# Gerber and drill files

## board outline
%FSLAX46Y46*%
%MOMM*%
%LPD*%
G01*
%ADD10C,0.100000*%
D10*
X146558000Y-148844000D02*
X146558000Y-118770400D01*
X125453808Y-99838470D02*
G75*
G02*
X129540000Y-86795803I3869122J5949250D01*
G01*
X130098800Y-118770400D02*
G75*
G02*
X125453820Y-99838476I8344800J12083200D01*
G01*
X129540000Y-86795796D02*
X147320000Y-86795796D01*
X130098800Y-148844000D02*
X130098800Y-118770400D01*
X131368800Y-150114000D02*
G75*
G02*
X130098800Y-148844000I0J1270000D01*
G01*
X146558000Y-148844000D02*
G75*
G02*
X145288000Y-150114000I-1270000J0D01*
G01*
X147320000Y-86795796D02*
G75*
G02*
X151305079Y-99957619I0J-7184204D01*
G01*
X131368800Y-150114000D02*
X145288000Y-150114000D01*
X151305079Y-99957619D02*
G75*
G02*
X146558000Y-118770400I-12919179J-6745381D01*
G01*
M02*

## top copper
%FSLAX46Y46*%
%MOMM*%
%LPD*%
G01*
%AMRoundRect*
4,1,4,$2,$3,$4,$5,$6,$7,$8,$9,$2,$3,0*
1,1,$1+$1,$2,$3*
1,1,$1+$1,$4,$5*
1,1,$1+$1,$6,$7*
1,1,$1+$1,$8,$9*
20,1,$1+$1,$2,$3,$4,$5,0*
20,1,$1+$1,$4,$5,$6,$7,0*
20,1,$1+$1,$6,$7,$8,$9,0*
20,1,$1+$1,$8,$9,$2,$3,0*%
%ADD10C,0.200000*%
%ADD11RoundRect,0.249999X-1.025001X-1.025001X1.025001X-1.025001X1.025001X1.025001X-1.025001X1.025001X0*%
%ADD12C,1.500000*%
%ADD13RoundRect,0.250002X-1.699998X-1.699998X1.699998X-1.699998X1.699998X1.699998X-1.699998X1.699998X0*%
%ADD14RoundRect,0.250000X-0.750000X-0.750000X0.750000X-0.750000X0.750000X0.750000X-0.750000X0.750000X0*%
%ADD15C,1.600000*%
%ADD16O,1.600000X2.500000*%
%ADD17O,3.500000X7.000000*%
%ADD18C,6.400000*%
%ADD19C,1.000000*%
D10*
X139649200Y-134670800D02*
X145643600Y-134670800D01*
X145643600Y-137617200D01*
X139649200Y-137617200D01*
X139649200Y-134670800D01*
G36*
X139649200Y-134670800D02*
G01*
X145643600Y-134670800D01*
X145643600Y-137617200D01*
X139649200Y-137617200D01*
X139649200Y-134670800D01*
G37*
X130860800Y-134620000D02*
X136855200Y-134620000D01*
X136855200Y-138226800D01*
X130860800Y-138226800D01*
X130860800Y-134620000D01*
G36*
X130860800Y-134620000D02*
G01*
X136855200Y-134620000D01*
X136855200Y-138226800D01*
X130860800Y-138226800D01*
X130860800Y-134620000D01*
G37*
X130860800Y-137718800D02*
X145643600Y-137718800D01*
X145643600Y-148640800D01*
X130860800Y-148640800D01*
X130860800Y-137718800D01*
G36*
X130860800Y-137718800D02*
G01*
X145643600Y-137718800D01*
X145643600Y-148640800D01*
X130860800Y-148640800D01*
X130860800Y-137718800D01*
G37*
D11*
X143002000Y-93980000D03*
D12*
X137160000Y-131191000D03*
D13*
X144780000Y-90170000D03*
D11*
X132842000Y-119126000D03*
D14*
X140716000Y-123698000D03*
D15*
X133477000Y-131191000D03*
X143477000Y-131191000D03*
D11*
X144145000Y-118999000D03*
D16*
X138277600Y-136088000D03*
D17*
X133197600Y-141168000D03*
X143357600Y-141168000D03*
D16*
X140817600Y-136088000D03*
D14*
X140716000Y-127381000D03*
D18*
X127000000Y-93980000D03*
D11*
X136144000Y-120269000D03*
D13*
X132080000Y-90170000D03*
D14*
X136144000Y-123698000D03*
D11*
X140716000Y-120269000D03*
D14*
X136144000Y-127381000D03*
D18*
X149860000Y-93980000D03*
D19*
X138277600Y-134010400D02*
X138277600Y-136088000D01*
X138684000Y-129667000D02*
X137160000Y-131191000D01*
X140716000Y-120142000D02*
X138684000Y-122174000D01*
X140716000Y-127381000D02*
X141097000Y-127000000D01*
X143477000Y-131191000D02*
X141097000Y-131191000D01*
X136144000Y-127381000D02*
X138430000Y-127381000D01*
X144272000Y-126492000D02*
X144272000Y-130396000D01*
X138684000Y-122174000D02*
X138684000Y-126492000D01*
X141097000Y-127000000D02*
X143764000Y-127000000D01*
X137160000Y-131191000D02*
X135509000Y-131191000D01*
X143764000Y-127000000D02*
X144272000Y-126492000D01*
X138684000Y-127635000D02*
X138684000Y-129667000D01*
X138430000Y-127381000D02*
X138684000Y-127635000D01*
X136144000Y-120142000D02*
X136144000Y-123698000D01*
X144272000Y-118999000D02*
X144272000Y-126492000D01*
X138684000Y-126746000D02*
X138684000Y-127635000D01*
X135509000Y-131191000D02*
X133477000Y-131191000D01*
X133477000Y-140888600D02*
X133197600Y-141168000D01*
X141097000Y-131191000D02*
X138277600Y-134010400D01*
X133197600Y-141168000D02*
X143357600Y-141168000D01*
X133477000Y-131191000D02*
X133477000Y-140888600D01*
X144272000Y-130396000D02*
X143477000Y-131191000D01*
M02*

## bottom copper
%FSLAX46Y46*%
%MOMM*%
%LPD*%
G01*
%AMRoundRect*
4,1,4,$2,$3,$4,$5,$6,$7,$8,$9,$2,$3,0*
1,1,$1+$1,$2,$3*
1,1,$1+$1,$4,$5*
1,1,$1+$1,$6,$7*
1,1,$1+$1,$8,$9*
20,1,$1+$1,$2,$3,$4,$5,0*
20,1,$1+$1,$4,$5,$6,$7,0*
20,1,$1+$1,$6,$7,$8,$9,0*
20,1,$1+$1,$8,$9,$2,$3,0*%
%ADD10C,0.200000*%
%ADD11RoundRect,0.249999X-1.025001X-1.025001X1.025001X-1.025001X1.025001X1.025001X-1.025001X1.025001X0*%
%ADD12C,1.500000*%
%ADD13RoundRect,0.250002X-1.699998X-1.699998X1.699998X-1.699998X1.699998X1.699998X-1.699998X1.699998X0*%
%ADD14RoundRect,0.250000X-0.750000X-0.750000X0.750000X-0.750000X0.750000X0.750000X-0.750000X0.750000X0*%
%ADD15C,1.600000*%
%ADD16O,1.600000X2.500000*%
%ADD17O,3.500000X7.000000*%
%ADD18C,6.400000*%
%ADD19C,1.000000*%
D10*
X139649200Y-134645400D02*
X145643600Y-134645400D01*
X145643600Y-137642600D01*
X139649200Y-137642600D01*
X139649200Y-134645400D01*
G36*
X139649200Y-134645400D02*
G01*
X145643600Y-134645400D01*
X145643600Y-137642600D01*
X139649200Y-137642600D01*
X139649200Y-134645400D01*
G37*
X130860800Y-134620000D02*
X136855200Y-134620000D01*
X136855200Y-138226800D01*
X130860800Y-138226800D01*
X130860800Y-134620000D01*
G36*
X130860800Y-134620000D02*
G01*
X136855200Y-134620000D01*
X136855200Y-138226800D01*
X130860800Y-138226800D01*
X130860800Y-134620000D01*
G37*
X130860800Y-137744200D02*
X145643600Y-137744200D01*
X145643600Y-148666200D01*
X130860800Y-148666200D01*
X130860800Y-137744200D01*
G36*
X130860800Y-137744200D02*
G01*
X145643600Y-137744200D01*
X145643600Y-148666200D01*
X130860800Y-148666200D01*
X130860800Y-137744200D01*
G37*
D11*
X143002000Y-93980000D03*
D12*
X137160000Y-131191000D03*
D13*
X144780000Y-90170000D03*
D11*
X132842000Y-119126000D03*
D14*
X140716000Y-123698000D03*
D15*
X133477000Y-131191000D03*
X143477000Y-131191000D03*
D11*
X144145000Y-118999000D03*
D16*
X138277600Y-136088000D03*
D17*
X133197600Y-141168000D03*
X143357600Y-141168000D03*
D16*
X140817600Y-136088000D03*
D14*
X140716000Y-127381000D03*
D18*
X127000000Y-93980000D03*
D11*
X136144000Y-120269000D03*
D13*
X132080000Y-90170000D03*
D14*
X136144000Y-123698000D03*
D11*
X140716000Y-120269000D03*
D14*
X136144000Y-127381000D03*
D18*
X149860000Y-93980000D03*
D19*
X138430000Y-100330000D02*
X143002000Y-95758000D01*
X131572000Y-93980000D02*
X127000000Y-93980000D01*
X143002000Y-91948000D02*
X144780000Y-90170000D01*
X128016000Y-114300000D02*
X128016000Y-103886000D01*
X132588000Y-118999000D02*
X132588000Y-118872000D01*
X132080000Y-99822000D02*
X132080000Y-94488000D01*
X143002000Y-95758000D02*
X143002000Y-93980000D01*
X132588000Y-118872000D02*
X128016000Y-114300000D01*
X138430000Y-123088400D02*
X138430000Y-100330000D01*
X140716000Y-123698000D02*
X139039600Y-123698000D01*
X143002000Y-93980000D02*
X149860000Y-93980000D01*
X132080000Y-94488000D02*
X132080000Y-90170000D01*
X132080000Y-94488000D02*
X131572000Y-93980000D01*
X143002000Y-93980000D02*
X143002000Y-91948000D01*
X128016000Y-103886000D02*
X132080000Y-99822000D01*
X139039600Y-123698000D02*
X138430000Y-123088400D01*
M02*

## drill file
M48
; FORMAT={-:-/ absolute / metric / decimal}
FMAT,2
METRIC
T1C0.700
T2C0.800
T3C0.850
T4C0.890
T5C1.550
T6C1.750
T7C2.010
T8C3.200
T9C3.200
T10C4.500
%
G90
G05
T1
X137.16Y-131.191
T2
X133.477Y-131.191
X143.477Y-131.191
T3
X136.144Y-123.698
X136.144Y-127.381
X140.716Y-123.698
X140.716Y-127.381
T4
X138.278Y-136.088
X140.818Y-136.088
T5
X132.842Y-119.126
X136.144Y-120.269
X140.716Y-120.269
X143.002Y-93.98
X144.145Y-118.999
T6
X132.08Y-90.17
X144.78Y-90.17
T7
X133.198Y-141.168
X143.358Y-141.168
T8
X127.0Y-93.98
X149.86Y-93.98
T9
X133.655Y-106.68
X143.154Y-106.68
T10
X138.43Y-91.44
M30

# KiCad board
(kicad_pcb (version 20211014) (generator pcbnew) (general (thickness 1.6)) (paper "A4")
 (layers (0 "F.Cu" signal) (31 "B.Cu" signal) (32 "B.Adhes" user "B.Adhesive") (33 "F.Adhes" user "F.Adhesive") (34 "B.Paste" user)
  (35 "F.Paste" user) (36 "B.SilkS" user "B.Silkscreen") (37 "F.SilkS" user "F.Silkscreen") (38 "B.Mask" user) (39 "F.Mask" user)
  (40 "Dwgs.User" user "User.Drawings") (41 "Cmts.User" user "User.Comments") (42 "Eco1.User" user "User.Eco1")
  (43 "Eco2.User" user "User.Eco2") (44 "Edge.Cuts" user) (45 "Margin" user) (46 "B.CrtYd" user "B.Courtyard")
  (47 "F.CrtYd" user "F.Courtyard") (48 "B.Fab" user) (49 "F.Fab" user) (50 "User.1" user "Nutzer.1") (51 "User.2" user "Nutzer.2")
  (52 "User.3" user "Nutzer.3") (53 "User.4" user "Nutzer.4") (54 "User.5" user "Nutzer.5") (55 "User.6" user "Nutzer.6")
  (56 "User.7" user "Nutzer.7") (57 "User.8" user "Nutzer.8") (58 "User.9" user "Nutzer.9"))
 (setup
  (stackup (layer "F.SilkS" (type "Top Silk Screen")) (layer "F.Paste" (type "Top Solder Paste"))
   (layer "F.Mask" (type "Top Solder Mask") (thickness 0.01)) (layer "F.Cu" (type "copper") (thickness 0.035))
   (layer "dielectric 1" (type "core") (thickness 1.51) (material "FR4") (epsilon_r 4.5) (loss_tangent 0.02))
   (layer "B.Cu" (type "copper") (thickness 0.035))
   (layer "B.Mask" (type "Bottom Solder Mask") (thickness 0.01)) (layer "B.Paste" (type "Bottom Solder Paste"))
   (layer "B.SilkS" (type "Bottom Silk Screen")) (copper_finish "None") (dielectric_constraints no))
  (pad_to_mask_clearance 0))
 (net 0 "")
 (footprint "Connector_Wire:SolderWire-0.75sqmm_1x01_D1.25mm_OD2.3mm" (layer "F.Cu") (at 143.002 93.98)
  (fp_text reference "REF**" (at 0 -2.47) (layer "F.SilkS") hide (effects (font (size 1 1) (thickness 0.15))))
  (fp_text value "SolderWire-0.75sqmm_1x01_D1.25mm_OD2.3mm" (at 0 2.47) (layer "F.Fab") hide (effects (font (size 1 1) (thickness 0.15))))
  (pad "1" thru_hole roundrect (at 0 0) (size 2.55 2.55) (drill 1.55) (layers *.Cu *.Mask) (roundrect_rratio 0.098039)))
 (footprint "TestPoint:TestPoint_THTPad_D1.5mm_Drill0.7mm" (layer "F.Cu") (at 137.16 131.191)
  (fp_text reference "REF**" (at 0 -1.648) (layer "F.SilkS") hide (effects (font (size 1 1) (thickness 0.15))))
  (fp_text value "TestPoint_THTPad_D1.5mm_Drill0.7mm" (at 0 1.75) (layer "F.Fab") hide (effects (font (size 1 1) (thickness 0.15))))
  (pad "1" thru_hole circle (at 0 0) (size 1.5 1.5) (drill 0.7) (layers *.Cu *.Mask)))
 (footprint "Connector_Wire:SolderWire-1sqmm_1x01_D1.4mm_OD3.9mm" (layer "F.Cu") (at 144.78 90.17)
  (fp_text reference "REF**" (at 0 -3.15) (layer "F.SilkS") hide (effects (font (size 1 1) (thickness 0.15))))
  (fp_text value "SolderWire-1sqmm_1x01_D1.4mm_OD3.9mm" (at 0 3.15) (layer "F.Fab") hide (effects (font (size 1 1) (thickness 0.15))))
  (pad "1" thru_hole roundrect (at 0 0) (size 3.9 3.9) (drill 1.75) (layers *.Cu *.Mask) (roundrect_rratio 0.064103)))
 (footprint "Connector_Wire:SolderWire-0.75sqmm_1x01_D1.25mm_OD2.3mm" (layer "F.Cu") (at 132.842 119.126)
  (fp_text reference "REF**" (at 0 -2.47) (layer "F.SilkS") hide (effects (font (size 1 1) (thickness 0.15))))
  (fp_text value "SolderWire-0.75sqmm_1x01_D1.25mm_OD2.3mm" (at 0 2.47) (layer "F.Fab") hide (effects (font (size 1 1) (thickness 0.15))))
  (pad "1" thru_hole roundrect (at 0 0) (size 2.55 2.55) (drill 1.55) (layers *.Cu *.Mask) (roundrect_rratio 0.098039)))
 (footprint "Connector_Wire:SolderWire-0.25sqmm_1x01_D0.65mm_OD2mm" (layer "F.Cu") (at 140.716 123.698)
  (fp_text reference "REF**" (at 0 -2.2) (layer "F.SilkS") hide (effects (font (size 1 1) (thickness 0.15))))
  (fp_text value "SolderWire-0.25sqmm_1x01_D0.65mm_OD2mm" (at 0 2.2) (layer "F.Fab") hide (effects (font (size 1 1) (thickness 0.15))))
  (pad "1" thru_hole roundrect (at 0 0) (size 2 2) (drill 0.85) (layers *.Cu *.Mask) (roundrect_rratio 0.125)))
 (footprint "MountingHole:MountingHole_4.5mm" (layer "F.Cu") (at 138.43 91.44)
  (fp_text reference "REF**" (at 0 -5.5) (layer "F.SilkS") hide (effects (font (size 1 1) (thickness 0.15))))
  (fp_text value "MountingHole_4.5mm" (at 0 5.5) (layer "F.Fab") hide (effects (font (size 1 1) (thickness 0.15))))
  (pad "" np_thru_hole circle (at 0 0) (size 4.5 4.5) (drill 4.5) (layers *.Cu *.Mask)))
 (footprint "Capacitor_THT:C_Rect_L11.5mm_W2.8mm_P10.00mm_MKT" (layer "F.Cu") (at 133.477 131.191)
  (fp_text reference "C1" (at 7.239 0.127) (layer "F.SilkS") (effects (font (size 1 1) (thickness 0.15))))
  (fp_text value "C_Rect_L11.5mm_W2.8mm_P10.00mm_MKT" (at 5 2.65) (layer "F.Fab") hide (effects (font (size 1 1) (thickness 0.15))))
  (pad "1" thru_hole circle (at 0 0) (size 1.6 1.6) (drill 0.8) (layers *.Cu *.Mask))
  (pad "2" thru_hole circle (at 10 0) (size 1.6 1.6) (drill 0.8) (layers *.Cu *.Mask)))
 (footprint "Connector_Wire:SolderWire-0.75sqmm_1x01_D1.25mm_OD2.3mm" (layer "F.Cu") (at 144.145 118.999)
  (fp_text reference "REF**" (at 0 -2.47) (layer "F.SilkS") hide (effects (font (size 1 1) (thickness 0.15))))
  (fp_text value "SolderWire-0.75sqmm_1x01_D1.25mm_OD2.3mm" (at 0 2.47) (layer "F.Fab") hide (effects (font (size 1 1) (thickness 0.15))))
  (pad "1" thru_hole roundrect (at 0 0) (size 2.55 2.55) (drill 1.55) (layers *.Cu *.Mask) (roundrect_rratio 0.098039)))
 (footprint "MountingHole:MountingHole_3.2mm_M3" (layer "F.Cu") (at 143.1544 106.68)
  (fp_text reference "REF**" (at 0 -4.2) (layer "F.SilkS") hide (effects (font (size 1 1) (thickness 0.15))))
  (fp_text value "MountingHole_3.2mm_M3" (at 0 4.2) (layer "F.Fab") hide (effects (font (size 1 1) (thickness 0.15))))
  (pad "" np_thru_hole circle (at 0 0) (size 3.2 3.2) (drill 3.2) (layers *.Cu *.Mask)))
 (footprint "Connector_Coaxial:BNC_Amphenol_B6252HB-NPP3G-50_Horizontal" (layer "F.Cu") (at 138.2776 136.088 180)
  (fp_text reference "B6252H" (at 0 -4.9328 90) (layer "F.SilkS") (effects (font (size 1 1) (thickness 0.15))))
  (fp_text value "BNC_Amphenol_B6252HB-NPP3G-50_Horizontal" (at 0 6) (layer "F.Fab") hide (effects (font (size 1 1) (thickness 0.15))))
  (pad "1" thru_hole oval (at 0 0 180) (size 1.6 2.5) (drill 0.89) (layers *.Cu *.Mask))
  (pad "2" thru_hole oval (at 5.08 -5.08 180) (size 3.5 7) (drill 2.01) (layers *.Cu *.Mask))
  (pad "2" thru_hole oval (at -5.08 -5.08 180) (size 3.5 7) (drill 2.01) (layers *.Cu *.Mask))
  (pad "2" thru_hole oval (at -2.54 0 180) (size 1.6 2.5) (drill 0.89) (layers *.Cu *.Mask)))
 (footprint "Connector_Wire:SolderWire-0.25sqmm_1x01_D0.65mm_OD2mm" (layer "F.Cu") (at 140.716 127.381)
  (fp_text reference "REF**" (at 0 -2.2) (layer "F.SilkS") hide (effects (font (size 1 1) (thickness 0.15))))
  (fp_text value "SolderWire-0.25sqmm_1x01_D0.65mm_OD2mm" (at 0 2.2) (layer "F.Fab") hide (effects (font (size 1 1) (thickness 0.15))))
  (pad "1" thru_hole roundrect (at 0 0) (size 2 2) (drill 0.85) (layers *.Cu *.Mask) (roundrect_rratio 0.125)))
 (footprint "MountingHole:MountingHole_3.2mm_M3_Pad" (layer "F.Cu") (at 127 93.98)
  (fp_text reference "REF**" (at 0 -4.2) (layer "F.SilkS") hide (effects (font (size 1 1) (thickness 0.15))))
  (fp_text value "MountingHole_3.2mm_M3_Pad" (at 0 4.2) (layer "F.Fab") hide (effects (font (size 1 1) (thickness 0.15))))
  (pad "1" thru_hole circle (at 0 0) (size 6.4 6.4) (drill 3.2) (layers *.Cu *.Mask)))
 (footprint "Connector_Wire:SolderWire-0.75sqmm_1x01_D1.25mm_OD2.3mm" (layer "F.Cu") (at 136.144 120.269)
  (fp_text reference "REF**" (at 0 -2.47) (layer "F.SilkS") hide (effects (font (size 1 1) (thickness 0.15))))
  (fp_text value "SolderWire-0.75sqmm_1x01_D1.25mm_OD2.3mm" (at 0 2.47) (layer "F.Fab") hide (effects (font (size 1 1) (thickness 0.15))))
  (pad "1" thru_hole roundrect (at 0 0) (size 2.55 2.55) (drill 1.55) (layers *.Cu *.Mask) (roundrect_rratio 0.098039)))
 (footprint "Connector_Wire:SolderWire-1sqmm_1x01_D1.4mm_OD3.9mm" (layer "F.Cu") (at 132.08 90.17)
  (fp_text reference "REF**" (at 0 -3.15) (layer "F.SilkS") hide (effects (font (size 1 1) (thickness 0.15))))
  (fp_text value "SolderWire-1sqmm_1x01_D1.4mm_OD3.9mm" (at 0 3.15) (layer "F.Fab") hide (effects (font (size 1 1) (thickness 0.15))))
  (pad "1" thru_hole roundrect (at 0 0) (size 3.9 3.9) (drill 1.75) (layers *.Cu *.Mask) (roundrect_rratio 0.064103)))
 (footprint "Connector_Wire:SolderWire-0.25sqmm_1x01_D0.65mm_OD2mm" (layer "F.Cu") (at 136.144 123.698)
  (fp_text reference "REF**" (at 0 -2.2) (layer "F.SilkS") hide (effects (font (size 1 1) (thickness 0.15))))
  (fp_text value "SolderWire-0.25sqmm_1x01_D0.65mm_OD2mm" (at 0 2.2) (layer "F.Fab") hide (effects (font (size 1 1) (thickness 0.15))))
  (pad "1" thru_hole roundrect (at 0 0) (size 2 2) (drill 0.85) (layers *.Cu *.Mask) (roundrect_rratio 0.125)))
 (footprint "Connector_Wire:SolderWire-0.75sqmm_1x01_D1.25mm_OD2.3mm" (layer "F.Cu") (at 140.716 120.269)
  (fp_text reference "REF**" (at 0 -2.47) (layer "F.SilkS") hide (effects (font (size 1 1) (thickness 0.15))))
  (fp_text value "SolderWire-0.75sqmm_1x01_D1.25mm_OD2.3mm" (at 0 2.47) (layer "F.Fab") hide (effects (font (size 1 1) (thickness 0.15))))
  (pad "1" thru_hole roundrect (at 0 0) (size 2.55 2.55) (drill 1.55) (layers *.Cu *.Mask) (roundrect_rratio 0.098039)))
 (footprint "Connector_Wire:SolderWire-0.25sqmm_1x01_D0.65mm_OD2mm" (layer "F.Cu") (at 136.144 127.381)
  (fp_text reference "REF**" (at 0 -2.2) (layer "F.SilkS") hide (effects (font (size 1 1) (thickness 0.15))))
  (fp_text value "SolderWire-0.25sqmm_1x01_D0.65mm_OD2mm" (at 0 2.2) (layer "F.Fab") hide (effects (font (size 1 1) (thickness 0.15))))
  (pad "1" thru_hole roundrect (at 0 0) (size 2 2) (drill 0.85) (layers *.Cu *.Mask) (roundrect_rratio 0.125)))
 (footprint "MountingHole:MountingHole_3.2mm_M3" (layer "F.Cu") (at 133.6548 106.68)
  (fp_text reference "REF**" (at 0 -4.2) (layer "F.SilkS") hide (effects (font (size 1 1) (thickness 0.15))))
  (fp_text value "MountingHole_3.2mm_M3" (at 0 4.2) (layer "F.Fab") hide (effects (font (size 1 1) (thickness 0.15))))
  (pad "" np_thru_hole circle (at 0 0) (size 3.2 3.2) (drill 3.2) (layers *.Cu *.Mask)))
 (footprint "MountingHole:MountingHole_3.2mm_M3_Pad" (layer "F.Cu") (at 149.86 93.98)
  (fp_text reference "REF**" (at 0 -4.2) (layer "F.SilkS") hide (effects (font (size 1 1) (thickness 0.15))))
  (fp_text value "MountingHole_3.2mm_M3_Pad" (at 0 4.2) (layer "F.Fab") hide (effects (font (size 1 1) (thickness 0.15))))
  (pad "1" thru_hole circle (at 0 0) (size 6.4 6.4) (drill 3.2) (layers *.Cu *.Mask)))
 (gr_rect (start 145.6436 134.6708) (end 139.6492 137.6172) (layer "F.Cu") (width 0.2) (fill solid))
 (gr_rect (start 136.8552 134.62) (end 130.8608 138.2268) (layer "F.Cu") (width 0.2) (fill solid))
 (gr_rect (start 145.6436 137.7188) (end 130.8608 148.6408) (layer "F.Cu") (width 0.2) (fill solid))
 (gr_rect (start 145.6436 134.6454) (end 139.6492 137.6426) (layer "B.Cu") (width 0.2) (fill solid))
 (gr_rect (start 136.8552 134.62) (end 130.8608 138.2268) (layer "B.Cu") (width 0.2) (fill solid))
 (gr_rect (start 145.6436 137.7442) (end 130.8608 148.6662) (layer "B.Cu") (width 0.2) (fill solid))
 (gr_line (start 146.558 148.844) (end 146.558 118.7704) (layer "Edge.Cuts") (width 0.1))
 (gr_arc (start 125.453808 99.83847) (mid 122.550769 91.767538) (end 129.54 86.795796) (layer "Edge.Cuts") (width 0.1))
 (gr_arc (start 130.0988 118.7704) (mid 124.181921 110.186325) (end 125.453808 99.83847) (layer "Edge.Cuts") (width 0.1))
 (gr_line (start 129.54 86.795796) (end 147.32 86.795796) (layer "Edge.Cuts") (width 0.1))
 (gr_line (start 130.0988 148.844) (end 130.0988 118.7704) (layer "Edge.Cuts") (width 0.1))
 (gr_arc (start 131.3688 150.114) (mid 130.470774 149.742026) (end 130.0988 148.844) (layer "Edge.Cuts") (width 0.1))
 (gr_arc (start 146.558 148.844) (mid 146.186026 149.742026) (end 145.288 150.114) (layer "Edge.Cuts") (width 0.1))
 (gr_arc (start 147.32 86.795796) (mid 154.195942 91.898132) (end 151.305079 99.957619) (layer "Edge.Cuts") (width 0.1))
 (gr_line (start 131.3688 150.114) (end 145.288 150.114) (layer "Edge.Cuts") (width 0.1))
 (gr_arc (start 151.305079 99.957619) (mid 152.5171 110.268764) (end 146.558 118.7704) (layer "Edge.Cuts") (width 0.1))
 (segment (start 138.2776 134.0104) (end 138.2776 136.088) (width 1) (layer "F.Cu") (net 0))
 (segment (start 138.684 129.667) (end 137.16 131.191) (width 1) (layer "F.Cu") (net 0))
 (segment (start 140.716 120.142) (end 138.684 122.174) (width 1) (layer "F.Cu") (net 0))
 (segment (start 140.716 127.381) (end 141.097 127) (width 1) (layer "F.Cu") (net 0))
 (segment (start 143.477 131.191) (end 141.097 131.191) (width 1) (layer "F.Cu") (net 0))
 (segment (start 136.144 127.381) (end 138.43 127.381) (width 1) (layer "F.Cu") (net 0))
 (segment (start 144.272 126.492) (end 144.272 130.396) (width 1) (layer "F.Cu") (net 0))
 (segment (start 138.684 122.174) (end 138.684 126.492) (width 1) (layer "F.Cu") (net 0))
 (segment (start 141.097 127) (end 143.764 127) (width 1) (layer "F.Cu") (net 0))
 (segment (start 137.16 131.191) (end 135.509 131.191) (width 1) (layer "F.Cu") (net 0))
 (segment (start 143.764 127) (end 144.272 126.492) (width 1) (layer "F.Cu") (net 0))
 (segment (start 138.684 127.635) (end 138.684 129.667) (width 1) (layer "F.Cu") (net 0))
 (segment (start 138.43 127.381) (end 138.684 127.635) (width 1) (layer "F.Cu") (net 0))
 (segment (start 136.144 120.142) (end 136.144 123.698) (width 1) (layer "F.Cu") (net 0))
 (segment (start 144.272 118.999) (end 144.272 126.492) (width 1) (layer "F.Cu") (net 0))
 (segment (start 138.684 126.746) (end 138.684 127.635) (width 1) (layer "F.Cu") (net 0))
 (segment (start 135.509 131.191) (end 133.477 131.191) (width 1) (layer "F.Cu") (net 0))
 (segment (start 133.477 140.8886) (end 133.1976 141.168) (width 1) (layer "F.Cu") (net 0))
 (segment (start 141.097 131.191) (end 138.2776 134.0104) (width 1) (layer "F.Cu") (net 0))
 (segment (start 133.1976 141.168) (end 143.3576 141.168) (width 1) (layer "F.Cu") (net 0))
 (segment (start 133.477 131.191) (end 133.477 140.8886) (width 1) (layer "F.Cu") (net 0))
 (segment (start 144.272 130.396) (end 143.477 131.191) (width 1) (layer "F.Cu") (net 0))
 (segment (start 138.43 100.33) (end 143.002 95.758) (width 1) (layer "B.Cu") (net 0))
 (segment (start 131.572 93.98) (end 127 93.98) (width 1) (layer "B.Cu") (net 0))
 (segment (start 143.002 91.948) (end 144.78 90.17) (width 1) (layer "B.Cu") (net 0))
 (segment (start 128.016 114.3) (end 128.016 103.886) (width 1) (layer "B.Cu") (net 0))
 (segment (start 132.588 118.999) (end 132.588 118.872) (width 1) (layer "B.Cu") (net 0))
 (segment (start 132.08 99.822) (end 132.08 94.488) (width 1) (layer "B.Cu") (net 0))
 (segment (start 143.002 95.758) (end 143.002 93.98) (width 1) (layer "B.Cu") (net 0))
 (segment (start 132.588 118.872) (end 128.016 114.3) (width 1) (layer "B.Cu") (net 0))
 (segment (start 138.43 123.0884) (end 138.43 100.33) (width 1) (layer "B.Cu") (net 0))
 (segment (start 140.716 123.698) (end 139.0396 123.698) (width 1) (layer "B.Cu") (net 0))
 (segment (start 143.002 93.98) (end 149.86 93.98) (width 1) (layer "B.Cu") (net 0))
 (segment (start 132.08 94.488) (end 132.08 90.17) (width 1) (layer "B.Cu") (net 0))
 (segment (start 132.08 94.488) (end 131.572 93.98) (width 1) (layer "B.Cu") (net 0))
 (segment (start 143.002 93.98) (end 143.002 91.948) (width 1) (layer "B.Cu") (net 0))
 (segment (start 128.016 103.886) (end 132.08 99.822) (width 1) (layer "B.Cu") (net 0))
 (segment (start 139.0396 123.698) (end 138.43 123.0884) (width 1) (layer "B.Cu") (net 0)))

